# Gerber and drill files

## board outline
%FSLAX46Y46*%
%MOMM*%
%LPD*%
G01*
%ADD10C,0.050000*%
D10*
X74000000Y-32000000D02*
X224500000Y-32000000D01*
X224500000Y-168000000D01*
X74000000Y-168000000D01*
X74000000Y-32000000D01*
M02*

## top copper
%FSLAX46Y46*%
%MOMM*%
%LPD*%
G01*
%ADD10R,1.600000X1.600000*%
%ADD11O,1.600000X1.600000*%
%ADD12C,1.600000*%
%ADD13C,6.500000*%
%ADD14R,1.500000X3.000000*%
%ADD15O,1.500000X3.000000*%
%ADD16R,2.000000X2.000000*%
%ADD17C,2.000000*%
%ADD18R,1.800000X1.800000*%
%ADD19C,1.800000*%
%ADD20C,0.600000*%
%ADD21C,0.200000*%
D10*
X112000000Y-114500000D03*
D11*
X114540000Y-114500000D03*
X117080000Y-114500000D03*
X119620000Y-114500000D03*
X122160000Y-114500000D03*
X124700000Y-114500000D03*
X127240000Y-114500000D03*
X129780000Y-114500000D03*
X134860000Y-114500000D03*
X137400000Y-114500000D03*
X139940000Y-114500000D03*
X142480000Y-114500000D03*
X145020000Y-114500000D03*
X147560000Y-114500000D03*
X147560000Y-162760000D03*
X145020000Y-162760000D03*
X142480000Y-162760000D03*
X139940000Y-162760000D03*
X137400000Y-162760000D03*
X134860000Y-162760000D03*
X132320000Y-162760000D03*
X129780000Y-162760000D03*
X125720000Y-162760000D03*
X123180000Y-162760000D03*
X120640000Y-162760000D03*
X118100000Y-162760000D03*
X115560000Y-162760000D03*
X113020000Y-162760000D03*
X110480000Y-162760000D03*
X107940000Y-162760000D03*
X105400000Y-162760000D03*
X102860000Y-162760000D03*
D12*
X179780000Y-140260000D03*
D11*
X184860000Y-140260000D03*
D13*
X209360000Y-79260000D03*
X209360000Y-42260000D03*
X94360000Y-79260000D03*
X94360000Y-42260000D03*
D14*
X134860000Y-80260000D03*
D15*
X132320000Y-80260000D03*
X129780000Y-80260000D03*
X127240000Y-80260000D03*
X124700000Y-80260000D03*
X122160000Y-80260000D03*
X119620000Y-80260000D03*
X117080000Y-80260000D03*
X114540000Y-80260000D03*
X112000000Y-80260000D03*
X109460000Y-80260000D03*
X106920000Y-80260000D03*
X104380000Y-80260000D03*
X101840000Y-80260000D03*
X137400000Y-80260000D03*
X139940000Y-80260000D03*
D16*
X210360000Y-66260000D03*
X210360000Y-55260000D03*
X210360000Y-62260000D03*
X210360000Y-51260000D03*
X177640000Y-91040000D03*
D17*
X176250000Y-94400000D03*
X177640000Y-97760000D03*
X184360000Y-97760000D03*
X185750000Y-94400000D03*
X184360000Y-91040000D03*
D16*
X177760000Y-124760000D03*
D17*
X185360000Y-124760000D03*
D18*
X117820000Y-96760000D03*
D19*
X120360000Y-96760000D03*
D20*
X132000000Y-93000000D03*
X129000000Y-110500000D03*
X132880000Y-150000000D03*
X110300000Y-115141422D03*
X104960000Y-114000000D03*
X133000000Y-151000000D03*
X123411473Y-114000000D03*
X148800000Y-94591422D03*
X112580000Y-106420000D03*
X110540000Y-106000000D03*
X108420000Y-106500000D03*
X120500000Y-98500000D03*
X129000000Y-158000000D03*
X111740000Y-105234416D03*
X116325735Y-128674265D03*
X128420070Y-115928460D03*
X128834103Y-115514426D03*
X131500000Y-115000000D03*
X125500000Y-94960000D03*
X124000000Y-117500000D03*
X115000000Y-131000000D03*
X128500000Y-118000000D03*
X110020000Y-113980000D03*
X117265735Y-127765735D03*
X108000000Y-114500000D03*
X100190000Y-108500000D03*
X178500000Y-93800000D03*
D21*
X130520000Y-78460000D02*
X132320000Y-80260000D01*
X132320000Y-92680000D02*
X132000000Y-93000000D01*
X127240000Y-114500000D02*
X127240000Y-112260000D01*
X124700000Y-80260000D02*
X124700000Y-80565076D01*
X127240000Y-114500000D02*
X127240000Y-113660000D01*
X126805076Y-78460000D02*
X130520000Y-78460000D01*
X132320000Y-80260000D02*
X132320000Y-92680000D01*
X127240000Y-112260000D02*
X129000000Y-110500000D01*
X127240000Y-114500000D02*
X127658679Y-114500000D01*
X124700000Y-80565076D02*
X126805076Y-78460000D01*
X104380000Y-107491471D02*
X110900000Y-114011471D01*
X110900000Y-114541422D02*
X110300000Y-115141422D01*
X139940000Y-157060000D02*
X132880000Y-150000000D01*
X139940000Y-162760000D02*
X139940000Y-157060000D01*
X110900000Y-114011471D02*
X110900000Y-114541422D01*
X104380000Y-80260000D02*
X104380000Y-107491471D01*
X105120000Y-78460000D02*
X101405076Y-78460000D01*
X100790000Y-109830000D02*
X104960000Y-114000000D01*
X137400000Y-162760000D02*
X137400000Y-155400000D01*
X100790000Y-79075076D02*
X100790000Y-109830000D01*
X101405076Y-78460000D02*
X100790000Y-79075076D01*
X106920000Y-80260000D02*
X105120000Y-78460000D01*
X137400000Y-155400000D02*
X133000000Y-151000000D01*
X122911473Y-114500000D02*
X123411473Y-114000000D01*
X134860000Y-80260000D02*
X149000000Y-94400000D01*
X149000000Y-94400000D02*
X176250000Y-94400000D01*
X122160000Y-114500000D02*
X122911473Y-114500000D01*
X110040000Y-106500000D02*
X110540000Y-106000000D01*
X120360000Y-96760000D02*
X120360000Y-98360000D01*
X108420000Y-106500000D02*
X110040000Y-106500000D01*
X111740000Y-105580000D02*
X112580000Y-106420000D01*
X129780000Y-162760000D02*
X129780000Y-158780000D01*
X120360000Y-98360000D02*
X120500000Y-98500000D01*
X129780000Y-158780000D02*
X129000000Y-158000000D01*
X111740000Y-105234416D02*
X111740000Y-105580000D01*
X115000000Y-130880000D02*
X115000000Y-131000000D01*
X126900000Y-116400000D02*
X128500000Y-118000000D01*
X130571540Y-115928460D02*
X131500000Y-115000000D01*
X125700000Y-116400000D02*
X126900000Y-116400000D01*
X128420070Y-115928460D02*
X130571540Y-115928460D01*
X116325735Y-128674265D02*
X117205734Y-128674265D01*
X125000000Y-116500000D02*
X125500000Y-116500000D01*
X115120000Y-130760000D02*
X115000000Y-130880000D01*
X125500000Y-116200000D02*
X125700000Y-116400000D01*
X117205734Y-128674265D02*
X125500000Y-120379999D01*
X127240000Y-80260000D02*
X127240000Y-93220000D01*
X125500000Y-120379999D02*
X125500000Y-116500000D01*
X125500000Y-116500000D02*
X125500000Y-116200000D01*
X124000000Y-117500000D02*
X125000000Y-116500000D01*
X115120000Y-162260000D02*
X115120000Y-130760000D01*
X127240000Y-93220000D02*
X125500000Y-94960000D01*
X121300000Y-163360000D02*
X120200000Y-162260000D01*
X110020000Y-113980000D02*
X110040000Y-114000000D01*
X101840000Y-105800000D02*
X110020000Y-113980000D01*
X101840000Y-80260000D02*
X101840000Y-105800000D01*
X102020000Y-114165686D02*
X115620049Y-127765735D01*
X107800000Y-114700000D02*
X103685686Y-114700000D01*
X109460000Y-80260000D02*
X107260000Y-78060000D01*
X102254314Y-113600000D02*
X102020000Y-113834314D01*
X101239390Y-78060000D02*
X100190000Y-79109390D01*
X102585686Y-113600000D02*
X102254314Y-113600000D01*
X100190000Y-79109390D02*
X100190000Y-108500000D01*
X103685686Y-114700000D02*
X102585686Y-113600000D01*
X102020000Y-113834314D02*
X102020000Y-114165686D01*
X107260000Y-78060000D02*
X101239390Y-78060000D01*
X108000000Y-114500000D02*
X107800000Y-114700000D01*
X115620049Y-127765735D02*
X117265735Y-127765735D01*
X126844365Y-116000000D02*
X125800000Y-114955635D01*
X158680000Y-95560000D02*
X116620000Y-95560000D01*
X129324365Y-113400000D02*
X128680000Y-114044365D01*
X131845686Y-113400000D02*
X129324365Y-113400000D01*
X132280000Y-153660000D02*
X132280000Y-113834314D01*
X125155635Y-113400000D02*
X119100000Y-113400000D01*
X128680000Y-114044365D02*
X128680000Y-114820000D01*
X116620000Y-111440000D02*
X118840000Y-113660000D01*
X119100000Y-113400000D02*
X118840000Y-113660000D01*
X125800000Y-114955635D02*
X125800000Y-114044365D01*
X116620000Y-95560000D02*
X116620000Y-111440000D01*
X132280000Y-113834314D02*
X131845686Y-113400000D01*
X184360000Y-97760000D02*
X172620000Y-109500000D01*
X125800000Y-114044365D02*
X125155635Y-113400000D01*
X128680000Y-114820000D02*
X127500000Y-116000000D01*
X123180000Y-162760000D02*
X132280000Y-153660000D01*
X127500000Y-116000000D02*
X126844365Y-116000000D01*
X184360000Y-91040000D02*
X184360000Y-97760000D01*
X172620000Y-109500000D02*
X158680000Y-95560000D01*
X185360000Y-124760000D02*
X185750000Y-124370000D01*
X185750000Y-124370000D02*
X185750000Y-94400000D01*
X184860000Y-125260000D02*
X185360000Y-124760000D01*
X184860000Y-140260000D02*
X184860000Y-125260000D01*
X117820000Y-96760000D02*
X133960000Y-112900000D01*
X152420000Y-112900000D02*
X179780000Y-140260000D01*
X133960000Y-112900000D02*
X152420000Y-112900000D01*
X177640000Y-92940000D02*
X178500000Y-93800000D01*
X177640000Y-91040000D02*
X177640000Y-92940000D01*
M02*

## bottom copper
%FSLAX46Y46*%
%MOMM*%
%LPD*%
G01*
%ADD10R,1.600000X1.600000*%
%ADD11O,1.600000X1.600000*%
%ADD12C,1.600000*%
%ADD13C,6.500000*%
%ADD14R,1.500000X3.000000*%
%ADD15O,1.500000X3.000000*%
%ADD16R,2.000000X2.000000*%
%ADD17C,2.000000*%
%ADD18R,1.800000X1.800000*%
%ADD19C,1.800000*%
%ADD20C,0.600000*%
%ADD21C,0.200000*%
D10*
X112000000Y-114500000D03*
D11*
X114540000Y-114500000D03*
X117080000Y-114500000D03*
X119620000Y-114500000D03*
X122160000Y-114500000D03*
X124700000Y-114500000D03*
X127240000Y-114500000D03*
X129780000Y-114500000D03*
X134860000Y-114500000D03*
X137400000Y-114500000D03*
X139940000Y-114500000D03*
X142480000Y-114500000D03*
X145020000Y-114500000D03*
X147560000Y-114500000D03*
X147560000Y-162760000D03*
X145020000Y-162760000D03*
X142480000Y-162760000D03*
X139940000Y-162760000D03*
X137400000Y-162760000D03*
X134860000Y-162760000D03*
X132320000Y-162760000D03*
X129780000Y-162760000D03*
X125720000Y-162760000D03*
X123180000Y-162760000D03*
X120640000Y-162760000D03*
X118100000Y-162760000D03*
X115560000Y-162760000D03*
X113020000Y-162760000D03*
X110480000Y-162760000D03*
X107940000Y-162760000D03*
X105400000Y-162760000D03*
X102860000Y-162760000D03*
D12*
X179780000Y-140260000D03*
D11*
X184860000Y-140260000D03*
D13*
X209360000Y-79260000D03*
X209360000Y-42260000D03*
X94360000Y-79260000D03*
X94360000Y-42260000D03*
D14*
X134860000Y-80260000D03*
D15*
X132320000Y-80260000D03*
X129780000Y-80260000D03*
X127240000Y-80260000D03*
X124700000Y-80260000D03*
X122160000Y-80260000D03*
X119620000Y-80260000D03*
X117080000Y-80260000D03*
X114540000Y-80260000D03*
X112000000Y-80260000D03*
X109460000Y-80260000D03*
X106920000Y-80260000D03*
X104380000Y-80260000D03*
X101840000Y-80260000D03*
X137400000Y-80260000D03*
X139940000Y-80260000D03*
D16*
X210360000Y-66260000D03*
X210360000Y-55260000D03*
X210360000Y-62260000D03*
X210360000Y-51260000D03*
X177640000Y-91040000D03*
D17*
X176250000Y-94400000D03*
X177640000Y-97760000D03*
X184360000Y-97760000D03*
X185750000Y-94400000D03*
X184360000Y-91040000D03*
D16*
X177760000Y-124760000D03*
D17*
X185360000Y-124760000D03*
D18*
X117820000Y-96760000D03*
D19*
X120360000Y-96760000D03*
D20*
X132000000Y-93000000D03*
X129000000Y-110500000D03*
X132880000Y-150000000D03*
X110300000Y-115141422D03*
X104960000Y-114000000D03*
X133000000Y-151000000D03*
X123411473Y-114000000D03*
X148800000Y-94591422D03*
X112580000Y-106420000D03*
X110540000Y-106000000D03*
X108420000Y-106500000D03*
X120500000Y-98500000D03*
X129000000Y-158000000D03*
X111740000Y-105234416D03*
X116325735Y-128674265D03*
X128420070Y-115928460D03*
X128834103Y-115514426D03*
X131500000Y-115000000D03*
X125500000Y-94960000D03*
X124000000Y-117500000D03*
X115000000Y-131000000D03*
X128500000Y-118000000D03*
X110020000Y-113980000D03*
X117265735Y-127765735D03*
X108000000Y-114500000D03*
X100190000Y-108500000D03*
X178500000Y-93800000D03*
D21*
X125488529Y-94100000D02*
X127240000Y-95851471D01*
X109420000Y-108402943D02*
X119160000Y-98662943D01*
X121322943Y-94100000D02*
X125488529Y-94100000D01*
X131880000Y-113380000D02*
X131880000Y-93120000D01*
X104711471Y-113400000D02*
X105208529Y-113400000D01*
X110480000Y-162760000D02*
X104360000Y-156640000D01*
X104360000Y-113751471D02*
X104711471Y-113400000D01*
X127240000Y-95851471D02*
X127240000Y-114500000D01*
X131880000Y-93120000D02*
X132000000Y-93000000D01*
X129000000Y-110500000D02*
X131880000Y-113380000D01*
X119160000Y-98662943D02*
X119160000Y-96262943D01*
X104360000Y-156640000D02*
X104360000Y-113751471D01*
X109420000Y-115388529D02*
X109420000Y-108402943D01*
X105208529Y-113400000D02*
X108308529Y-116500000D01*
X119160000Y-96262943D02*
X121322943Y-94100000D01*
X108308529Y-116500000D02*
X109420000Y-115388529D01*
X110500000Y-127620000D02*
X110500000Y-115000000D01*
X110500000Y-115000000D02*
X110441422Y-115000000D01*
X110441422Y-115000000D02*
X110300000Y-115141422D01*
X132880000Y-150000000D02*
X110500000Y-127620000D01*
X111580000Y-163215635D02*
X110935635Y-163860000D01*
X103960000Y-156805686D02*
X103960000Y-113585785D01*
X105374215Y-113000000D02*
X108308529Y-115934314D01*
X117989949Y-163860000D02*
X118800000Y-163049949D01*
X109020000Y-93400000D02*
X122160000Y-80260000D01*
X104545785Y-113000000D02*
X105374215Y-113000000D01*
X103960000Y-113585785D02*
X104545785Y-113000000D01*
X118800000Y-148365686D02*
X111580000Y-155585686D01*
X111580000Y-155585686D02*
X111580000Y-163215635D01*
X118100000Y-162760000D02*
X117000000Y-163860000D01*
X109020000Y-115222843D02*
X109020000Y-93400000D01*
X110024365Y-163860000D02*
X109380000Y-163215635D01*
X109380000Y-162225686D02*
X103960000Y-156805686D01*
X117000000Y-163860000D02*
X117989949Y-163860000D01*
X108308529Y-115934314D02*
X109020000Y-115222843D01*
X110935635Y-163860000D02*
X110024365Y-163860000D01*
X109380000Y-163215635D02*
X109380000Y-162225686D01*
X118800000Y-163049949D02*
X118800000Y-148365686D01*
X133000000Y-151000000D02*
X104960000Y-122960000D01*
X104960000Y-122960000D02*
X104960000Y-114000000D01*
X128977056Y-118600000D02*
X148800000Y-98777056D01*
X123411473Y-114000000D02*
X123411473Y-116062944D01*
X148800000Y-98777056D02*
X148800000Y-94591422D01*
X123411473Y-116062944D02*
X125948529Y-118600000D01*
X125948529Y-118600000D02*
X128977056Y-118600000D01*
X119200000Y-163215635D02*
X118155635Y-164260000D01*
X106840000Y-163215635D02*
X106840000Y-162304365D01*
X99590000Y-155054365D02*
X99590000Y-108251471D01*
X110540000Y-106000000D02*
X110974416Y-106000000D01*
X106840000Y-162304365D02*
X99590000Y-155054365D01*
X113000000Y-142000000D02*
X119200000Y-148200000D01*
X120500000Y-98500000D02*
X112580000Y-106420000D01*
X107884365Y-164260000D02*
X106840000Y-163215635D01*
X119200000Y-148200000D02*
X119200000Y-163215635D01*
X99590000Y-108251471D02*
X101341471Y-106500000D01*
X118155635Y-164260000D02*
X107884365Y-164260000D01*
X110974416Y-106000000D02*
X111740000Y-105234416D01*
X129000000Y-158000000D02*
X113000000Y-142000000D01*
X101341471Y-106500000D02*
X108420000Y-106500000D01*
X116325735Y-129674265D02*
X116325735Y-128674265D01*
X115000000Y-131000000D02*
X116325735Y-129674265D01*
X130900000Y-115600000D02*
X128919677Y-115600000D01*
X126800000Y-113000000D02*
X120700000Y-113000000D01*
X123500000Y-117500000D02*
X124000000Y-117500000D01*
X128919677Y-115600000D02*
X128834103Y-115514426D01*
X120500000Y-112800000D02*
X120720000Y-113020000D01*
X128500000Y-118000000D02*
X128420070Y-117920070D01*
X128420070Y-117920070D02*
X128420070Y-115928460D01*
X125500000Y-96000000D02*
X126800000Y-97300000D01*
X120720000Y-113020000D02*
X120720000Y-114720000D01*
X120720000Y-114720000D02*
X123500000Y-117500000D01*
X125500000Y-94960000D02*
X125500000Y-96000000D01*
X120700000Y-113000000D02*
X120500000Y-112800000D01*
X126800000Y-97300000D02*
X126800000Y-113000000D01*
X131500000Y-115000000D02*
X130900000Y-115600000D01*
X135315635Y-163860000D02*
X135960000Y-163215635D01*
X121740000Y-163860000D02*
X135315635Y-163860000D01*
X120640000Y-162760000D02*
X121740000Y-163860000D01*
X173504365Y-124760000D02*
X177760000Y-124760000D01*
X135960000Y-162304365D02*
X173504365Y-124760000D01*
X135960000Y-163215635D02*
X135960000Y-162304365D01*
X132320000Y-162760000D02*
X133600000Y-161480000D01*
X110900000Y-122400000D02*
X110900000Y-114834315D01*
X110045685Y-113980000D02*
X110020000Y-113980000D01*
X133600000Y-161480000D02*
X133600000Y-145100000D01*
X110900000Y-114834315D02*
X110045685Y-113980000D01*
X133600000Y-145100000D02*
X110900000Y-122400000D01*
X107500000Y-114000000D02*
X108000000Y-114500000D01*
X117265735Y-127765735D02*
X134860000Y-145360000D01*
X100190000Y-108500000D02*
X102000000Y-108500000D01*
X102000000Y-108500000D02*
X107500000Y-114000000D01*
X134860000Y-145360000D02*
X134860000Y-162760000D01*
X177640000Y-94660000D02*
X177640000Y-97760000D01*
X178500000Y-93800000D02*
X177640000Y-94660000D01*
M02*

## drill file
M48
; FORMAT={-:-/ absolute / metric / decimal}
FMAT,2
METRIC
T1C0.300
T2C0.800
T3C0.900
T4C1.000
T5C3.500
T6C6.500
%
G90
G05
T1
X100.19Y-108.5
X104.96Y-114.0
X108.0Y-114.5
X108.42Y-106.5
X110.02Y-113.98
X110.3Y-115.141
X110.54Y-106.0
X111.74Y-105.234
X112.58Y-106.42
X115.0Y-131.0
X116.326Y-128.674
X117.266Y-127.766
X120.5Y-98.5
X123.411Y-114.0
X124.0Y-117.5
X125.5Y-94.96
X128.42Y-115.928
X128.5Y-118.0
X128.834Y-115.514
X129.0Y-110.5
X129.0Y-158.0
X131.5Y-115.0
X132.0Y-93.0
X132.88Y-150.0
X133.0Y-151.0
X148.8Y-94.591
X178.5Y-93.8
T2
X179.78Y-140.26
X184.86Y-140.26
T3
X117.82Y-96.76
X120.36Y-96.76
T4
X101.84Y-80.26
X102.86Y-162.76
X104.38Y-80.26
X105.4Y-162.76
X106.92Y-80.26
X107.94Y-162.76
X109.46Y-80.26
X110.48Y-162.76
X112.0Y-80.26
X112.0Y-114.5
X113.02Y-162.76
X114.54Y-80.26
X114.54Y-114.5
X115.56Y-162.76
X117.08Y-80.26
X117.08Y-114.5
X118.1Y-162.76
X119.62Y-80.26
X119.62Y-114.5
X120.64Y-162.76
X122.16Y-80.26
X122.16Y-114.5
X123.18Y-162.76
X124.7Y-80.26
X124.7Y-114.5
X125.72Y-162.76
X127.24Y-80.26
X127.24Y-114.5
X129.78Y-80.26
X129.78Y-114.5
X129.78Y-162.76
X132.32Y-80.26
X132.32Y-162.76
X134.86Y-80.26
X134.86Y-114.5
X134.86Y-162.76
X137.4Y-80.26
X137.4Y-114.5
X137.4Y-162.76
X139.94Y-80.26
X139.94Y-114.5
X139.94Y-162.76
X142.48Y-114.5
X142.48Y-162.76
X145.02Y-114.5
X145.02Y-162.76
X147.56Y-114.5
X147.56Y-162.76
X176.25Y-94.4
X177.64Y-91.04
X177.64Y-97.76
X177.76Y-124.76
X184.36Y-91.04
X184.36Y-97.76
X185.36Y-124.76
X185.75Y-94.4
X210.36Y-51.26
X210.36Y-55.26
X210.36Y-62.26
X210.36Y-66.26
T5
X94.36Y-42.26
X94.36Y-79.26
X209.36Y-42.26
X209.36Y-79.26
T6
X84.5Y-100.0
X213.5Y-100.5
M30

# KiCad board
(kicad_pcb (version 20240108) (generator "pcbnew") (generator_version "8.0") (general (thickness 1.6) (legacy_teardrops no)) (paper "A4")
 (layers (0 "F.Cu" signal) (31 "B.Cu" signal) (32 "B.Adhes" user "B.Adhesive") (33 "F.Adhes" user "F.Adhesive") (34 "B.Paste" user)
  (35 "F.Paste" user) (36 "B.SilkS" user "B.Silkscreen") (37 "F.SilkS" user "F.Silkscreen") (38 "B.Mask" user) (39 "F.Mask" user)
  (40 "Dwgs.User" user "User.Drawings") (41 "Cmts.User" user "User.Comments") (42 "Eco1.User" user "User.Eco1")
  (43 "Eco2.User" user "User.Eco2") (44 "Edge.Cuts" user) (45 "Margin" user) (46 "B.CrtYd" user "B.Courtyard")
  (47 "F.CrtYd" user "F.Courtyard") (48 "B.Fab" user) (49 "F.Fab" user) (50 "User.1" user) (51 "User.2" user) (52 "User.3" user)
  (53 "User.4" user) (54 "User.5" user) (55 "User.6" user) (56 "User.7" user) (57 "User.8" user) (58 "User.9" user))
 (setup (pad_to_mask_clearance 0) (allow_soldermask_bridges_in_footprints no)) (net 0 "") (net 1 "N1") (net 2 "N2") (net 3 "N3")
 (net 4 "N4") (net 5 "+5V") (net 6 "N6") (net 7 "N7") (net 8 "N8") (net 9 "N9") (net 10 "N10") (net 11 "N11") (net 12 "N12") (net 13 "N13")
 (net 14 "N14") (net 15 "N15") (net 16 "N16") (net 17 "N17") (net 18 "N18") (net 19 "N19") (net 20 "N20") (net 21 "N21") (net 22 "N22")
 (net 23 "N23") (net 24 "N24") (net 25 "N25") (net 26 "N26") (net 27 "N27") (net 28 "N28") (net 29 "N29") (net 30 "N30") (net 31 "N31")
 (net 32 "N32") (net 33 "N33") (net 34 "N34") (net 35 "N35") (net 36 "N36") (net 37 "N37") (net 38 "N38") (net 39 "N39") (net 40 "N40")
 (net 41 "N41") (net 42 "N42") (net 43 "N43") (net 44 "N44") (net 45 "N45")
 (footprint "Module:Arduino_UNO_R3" (layer "F.Cu") (at 112 114.5)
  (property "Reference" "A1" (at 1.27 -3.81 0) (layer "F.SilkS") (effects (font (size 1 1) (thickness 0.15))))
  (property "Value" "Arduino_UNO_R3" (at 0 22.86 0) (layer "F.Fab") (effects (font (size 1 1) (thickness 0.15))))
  (pad "1" thru_hole rect (at 0 0 90) (size 1.6 1.6) (drill 1) (layers "*.Cu" "*.Mask") (remove_unused_layers no) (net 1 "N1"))
  (pad "2" thru_hole oval (at 2.54 0 90) (size 1.6 1.6) (drill 1) (layers "*.Cu" "*.Mask") (remove_unused_layers no) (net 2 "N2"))
  (pad "3" thru_hole oval (at 5.08 0 90) (size 1.6 1.6) (drill 1) (layers "*.Cu" "*.Mask") (remove_unused_layers no) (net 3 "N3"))
  (pad "4" thru_hole oval (at 7.62 0 90) (size 1.6 1.6) (drill 1) (layers "*.Cu" "*.Mask") (remove_unused_layers no) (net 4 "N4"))
  (pad "5" thru_hole oval (at 10.16 0 90) (size 1.6 1.6) (drill 1) (layers "*.Cu" "*.Mask") (remove_unused_layers no) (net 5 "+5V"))
  (pad "6" thru_hole oval (at 12.7 0 90) (size 1.6 1.6) (drill 1) (layers "*.Cu" "*.Mask") (remove_unused_layers no) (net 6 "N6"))
  (pad "7" thru_hole oval (at 15.24 0 90) (size 1.6 1.6) (drill 1) (layers "*.Cu" "*.Mask") (remove_unused_layers no) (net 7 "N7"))
  (pad "8" thru_hole oval (at 17.78 0 90) (size 1.6 1.6) (drill 1) (layers "*.Cu" "*.Mask") (remove_unused_layers no) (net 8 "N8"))
  (pad "9" thru_hole oval (at 22.86 0 90) (size 1.6 1.6) (drill 1) (layers "*.Cu" "*.Mask") (remove_unused_layers no) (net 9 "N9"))
  (pad "10" thru_hole oval (at 25.4 0 90) (size 1.6 1.6) (drill 1) (layers "*.Cu" "*.Mask") (remove_unused_layers no) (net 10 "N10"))
  (pad "11" thru_hole oval (at 27.94 0 90) (size 1.6 1.6) (drill 1) (layers "*.Cu" "*.Mask") (remove_unused_layers no) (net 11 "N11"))
  (pad "12" thru_hole oval (at 30.48 0 90) (size 1.6 1.6) (drill 1) (layers "*.Cu" "*.Mask") (remove_unused_layers no) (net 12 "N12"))
  (pad "13" thru_hole oval (at 33.02 0 90) (size 1.6 1.6) (drill 1) (layers "*.Cu" "*.Mask") (remove_unused_layers no) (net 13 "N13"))
  (pad "14" thru_hole oval (at 35.56 0 90) (size 1.6 1.6) (drill 1) (layers "*.Cu" "*.Mask") (remove_unused_layers no) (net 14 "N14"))
  (pad "15" thru_hole oval (at 35.56 48.26 90) (size 1.6 1.6) (drill 1) (layers "*.Cu" "*.Mask") (remove_unused_layers no) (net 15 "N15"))
  (pad "16" thru_hole oval (at 33.02 48.26 90) (size 1.6 1.6) (drill 1) (layers "*.Cu" "*.Mask") (remove_unused_layers no) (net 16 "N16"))
  (pad "17" thru_hole oval (at 30.48 48.26 90) (size 1.6 1.6) (drill 1) (layers "*.Cu" "*.Mask") (remove_unused_layers no) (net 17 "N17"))
  (pad "18" thru_hole oval (at 27.94 48.26 90) (size 1.6 1.6) (drill 1) (layers "*.Cu" "*.Mask") (remove_unused_layers no) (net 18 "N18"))
  (pad "19" thru_hole oval (at 25.4 48.26 90) (size 1.6 1.6) (drill 1) (layers "*.Cu" "*.Mask") (remove_unused_layers no) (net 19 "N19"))
  (pad "20" thru_hole oval (at 22.86 48.26 90) (size 1.6 1.6) (drill 1) (layers "*.Cu" "*.Mask") (remove_unused_layers no) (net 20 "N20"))
  (pad "21" thru_hole oval (at 20.32 48.26 90) (size 1.6 1.6) (drill 1) (layers "*.Cu" "*.Mask") (remove_unused_layers no) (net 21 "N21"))
  (pad "22" thru_hole oval (at 17.78 48.26 90) (size 1.6 1.6) (drill 1) (layers "*.Cu" "*.Mask") (remove_unused_layers no) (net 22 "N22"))
  (pad "23" thru_hole oval (at 13.72 48.26 90) (size 1.6 1.6) (drill 1) (layers "*.Cu" "*.Mask") (remove_unused_layers no) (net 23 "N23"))
  (pad "24" thru_hole oval (at 11.18 48.26 90) (size 1.6 1.6) (drill 1) (layers "*.Cu" "*.Mask") (remove_unused_layers no) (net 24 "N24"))
  (pad "25" thru_hole oval (at 8.64 48.26 90) (size 1.6 1.6) (drill 1) (layers "*.Cu" "*.Mask") (remove_unused_layers no) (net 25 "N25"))
  (pad "26" thru_hole oval (at 6.1 48.26 90) (size 1.6 1.6) (drill 1) (layers "*.Cu" "*.Mask") (remove_unused_layers no) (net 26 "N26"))
  (pad "27" thru_hole oval (at 3.56 48.26 90) (size 1.6 1.6) (drill 1) (layers "*.Cu" "*.Mask") (remove_unused_layers no) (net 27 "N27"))
  (pad "28" thru_hole oval (at 1.02 48.26 90) (size 1.6 1.6) (drill 1) (layers "*.Cu" "*.Mask") (remove_unused_layers no) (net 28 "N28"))
  (pad "29" thru_hole oval (at -1.52 48.26 90) (size 1.6 1.6) (drill 1) (layers "*.Cu" "*.Mask") (remove_unused_layers no) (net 7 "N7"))
  (pad "30" thru_hole oval (at -4.06 48.26 90) (size 1.6 1.6) (drill 1) (layers "*.Cu" "*.Mask") (remove_unused_layers no) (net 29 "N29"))
  (pad "31" thru_hole oval (at -6.6 48.26 90) (size 1.6 1.6) (drill 1) (layers "*.Cu" "*.Mask") (remove_unused_layers no) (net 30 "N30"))
  (pad "32" thru_hole oval (at -9.14 48.26 90) (size 1.6 1.6) (drill 1) (layers "*.Cu" "*.Mask") (remove_unused_layers no) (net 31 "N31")))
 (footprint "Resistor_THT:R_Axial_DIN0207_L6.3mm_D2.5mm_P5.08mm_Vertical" (layer "F.Cu") (at 179.78 140.26)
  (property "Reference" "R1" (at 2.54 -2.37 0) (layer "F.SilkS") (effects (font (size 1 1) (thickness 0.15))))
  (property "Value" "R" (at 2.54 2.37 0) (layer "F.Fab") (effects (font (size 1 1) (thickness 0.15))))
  (pad "1" thru_hole circle (at 0 0) (size 1.6 1.6) (drill 0.8) (layers "*.Cu" "*.Mask") (remove_unused_layers no) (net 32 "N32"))
  (pad "2" thru_hole oval (at 5.08 0) (size 1.6 1.6) (drill 0.8) (layers "*.Cu" "*.Mask") (remove_unused_layers no) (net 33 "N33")))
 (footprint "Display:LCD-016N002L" (layer "F.Cu") (at 134.86 80.26 180)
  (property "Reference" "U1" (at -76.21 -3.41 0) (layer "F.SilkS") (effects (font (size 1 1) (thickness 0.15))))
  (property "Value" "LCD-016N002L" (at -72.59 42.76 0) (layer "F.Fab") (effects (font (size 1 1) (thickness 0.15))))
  (pad "" thru_hole circle (at -74.5 1) (size 6.5 6.5) (drill 3.5) (layers "*.Cu" "*.Mask") (remove_unused_layers no))
  (pad "" thru_hole circle (at -74.5 38) (size 6.5 6.5) (drill 3.5) (layers "*.Cu" "*.Mask") (remove_unused_layers no))
  (pad "" thru_hole circle (at 40.5 1) (size 6.5 6.5) (drill 3.5) (layers "*.Cu" "*.Mask") (remove_unused_layers no))
  (pad "" thru_hole circle (at 40.5 38) (size 6.5 6.5) (drill 3.5) (layers "*.Cu" "*.Mask") (remove_unused_layers no))
  (pad "1" thru_hole rect (at 0 0) (size 1.5 3) (drill 1) (layers "*.Cu" "*.Mask") (remove_unused_layers no) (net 5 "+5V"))
  (pad "2" thru_hole oval (at 2.54 0) (size 1.5 3) (drill 1) (layers "*.Cu" "*.Mask") (remove_unused_layers no) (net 7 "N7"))
  (pad "3" thru_hole oval (at 5.08 0) (size 1.5 3) (drill 1) (layers "*.Cu" "*.Mask") (remove_unused_layers no) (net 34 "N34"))
  (pad "4" thru_hole oval (at 7.62 0) (size 1.5 3) (drill 1) (layers "*.Cu" "*.Mask") (remove_unused_layers no) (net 27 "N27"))
  (pad "5" thru_hole oval (at 10.16 0) (size 1.5 3) (drill 1) (layers "*.Cu" "*.Mask") (remove_unused_layers no) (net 7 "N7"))
  (pad "6" thru_hole oval (at 12.7 0) (size 1.5 3) (drill 1) (layers "*.Cu" "*.Mask") (remove_unused_layers no) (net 26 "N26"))
  (pad "7" thru_hole oval (at 15.24 0) (size 1.5 3) (drill 1) (layers "*.Cu" "*.Mask") (remove_unused_layers no) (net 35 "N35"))
  (pad "8" thru_hole oval (at 17.78 0) (size 1.5 3) (drill 1) (layers "*.Cu" "*.Mask") (remove_unused_layers no) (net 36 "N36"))
  (pad "9" thru_hole oval (at 20.32 0) (size 1.5 3) (drill 1) (layers "*.Cu" "*.Mask") (remove_unused_layers no) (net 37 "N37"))
  (pad "10" thru_hole oval (at 22.86 0) (size 1.5 3) (drill 1) (layers "*.Cu" "*.Mask") (remove_unused_layers no) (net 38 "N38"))
  (pad "11" thru_hole oval (at 25.4 0) (size 1.5 3) (drill 1) (layers "*.Cu" "*.Mask") (remove_unused_layers no) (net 20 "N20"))
  (pad "12" thru_hole oval (at 27.94 0) (size 1.5 3) (drill 1) (layers "*.Cu" "*.Mask") (remove_unused_layers no) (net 19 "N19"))
  (pad "13" thru_hole oval (at 30.48 0) (size 1.5 3) (drill 1) (layers "*.Cu" "*.Mask") (remove_unused_layers no) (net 18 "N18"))
  (pad "14" thru_hole oval (at 33.02 0) (size 1.5 3) (drill 1) (layers "*.Cu" "*.Mask") (remove_unused_layers no) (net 21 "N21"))
  (pad "15" thru_hole oval (at -2.54 0) (size 1.5 3) (drill 1) (layers "*.Cu" "*.Mask") (remove_unused_layers no) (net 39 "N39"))
  (pad "16" thru_hole oval (at -5.08 0) (size 1.5 3) (drill 1) (layers "*.Cu" "*.Mask") (remove_unused_layers no) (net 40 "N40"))
  (pad "A1" thru_hole rect (at -75.5 14) (size 2 2) (drill 1) (layers "*.Cu" "*.Mask") (remove_unused_layers no) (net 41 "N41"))
  (pad "A2" thru_hole rect (at -75.5 25) (size 2 2) (drill 1) (layers "*.Cu" "*.Mask") (remove_unused_layers no) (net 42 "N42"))
  (pad "K1" thru_hole rect (at -75.5 18) (size 2 2) (drill 1) (layers "*.Cu" "*.Mask") (remove_unused_layers no) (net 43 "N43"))
  (pad "K2" thru_hole rect (at -75.5 29) (size 2 2) (drill 1) (layers "*.Cu" "*.Mask") (remove_unused_layers no) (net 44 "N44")))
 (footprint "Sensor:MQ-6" (layer "F.Cu") (at 177.64 91.04)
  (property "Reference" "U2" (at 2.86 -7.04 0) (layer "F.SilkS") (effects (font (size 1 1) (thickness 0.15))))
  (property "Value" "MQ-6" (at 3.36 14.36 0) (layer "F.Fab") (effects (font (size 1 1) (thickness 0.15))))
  (pad "1" thru_hole rect (at 0 0) (size 2 2) (drill 1) (layers "*.Cu" "*.Mask") (remove_unused_layers no) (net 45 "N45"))
  (pad "2" thru_hole circle (at -1.39 3.36) (size 2 2) (drill 1) (layers "*.Cu" "*.Mask") (remove_unused_layers no) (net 5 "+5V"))
  (pad "3" thru_hole circle (at 0 6.72 90) (size 2 2) (drill 1) (layers "*.Cu" "*.Mask") (remove_unused_layers no) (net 45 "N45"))
  (pad "4" thru_hole circle (at 6.72 6.72 180) (size 2 2) (drill 1) (layers "*.Cu" "*.Mask") (remove_unused_layers no) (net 24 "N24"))
  (pad "5" thru_hole circle (at 8.11 3.36) (size 2 2) (drill 1) (layers "*.Cu" "*.Mask") (remove_unused_layers no) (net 33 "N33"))
  (pad "6" thru_hole circle (at 6.72 0 270) (size 2 2) (drill 1) (layers "*.Cu" "*.Mask") (remove_unused_layers no) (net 24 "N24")))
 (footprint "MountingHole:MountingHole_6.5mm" (layer "F.Cu") (at 213.5 100.5)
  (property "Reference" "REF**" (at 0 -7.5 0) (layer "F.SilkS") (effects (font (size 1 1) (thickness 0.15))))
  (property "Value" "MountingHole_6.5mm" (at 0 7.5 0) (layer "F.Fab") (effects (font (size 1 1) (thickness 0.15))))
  (pad "" np_thru_hole circle (at 0 0) (size 6.5 6.5) (drill 6.5) (layers "*.Cu" "*.Mask")))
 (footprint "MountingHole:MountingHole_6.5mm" (layer "F.Cu") (at 84.5 100)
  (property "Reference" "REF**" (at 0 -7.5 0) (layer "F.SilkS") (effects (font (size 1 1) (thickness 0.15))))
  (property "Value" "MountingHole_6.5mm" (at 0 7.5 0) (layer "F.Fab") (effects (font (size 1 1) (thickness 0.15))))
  (pad "" np_thru_hole circle (at 0 0) (size 6.5 6.5) (drill 6.5) (layers "*.Cu" "*.Mask")))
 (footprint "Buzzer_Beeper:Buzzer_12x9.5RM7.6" (layer "F.Cu") (at 177.76 124.76)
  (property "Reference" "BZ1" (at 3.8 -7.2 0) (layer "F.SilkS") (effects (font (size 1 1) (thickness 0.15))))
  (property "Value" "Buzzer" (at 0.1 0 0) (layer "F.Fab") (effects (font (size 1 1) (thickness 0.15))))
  (pad "1" thru_hole rect (at 0 0) (size 2 2) (drill 1) (layers "*.Cu" "*.Mask") (remove_unused_layers no) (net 25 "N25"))
  (pad "2" thru_hole circle (at 7.6 0) (size 2 2) (drill 1) (layers "*.Cu" "*.Mask") (remove_unused_layers no) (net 33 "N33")))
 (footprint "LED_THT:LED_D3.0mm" (layer "F.Cu") (at 117.82 96.76)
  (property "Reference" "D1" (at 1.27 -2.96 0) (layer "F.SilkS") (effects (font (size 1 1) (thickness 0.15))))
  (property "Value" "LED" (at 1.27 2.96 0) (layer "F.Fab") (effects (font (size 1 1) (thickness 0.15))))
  (pad "1" thru_hole rect (at 0 0) (size 1.8 1.8) (drill 0.9) (layers "*.Cu" "*.Mask") (remove_unused_layers no) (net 32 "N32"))
  (pad "2" thru_hole circle (at 2.54 0) (size 1.8 1.8) (drill 0.9) (layers "*.Cu" "*.Mask") (remove_unused_layers no) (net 22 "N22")))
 (gr_rect (start 74 32) (end 224.5 168) (stroke (width 0.05) (type default)) (fill none) (layer "Edge.Cuts"))
 (segment (start 130.52 78.46) (end 132.32 80.26) (width 0.2) (layer "F.Cu") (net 7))
 (segment (start 132.32 92.68) (end 132 93) (width 0.2) (layer "F.Cu") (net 7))
 (segment (start 127.24 114.5) (end 127.24 112.26) (width 0.2) (layer "F.Cu") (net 7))
 (segment (start 124.7 80.26) (end 124.7 80.565076) (width 0.2) (layer "F.Cu") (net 7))
 (segment (start 127.24 114.5) (end 127.24 113.66) (width 0.2) (layer "F.Cu") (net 7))
 (segment (start 126.805076 78.46) (end 130.52 78.46) (width 0.2) (layer "F.Cu") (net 7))
 (segment (start 132.32 80.26) (end 132.32 92.68) (width 0.2) (layer "F.Cu") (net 7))
 (segment (start 127.24 112.26) (end 129 110.5) (width 0.2) (layer "F.Cu") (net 7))
 (segment (start 127.24 114.5) (end 127.658679 114.5) (width 0.2) (layer "F.Cu") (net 7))
 (segment (start 124.7 80.565076) (end 126.805076 78.46) (width 0.2) (layer "F.Cu") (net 7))
 (via (at 132 93) (size 0.6) (drill 0.3) (layers "F.Cu" "B.Cu") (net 7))
 (via (at 129 110.5) (size 0.6) (drill 0.3) (layers "F.Cu" "B.Cu") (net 7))
 (segment (start 125.488529 94.1) (end 127.24 95.851471) (width 0.2) (layer "B.Cu") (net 7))
 (segment (start 109.42 108.402943) (end 119.16 98.662943) (width 0.2) (layer "B.Cu") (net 7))
 (segment (start 121.322943 94.1) (end 125.488529 94.1) (width 0.2) (layer "B.Cu") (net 7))
 (segment (start 131.88 113.38) (end 131.88 93.12) (width 0.2) (layer "B.Cu") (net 7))
 (segment (start 104.711471 113.4) (end 105.208529 113.4) (width 0.2) (layer "B.Cu") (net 7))
 (segment (start 110.48 162.76) (end 104.36 156.64) (width 0.2) (layer "B.Cu") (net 7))
 (segment (start 104.36 113.751471) (end 104.711471 113.4) (width 0.2) (layer "B.Cu") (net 7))
 (segment (start 127.24 95.851471) (end 127.24 114.5) (width 0.2) (layer "B.Cu") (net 7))
 (segment (start 131.88 93.12) (end 132 93) (width 0.2) (layer "B.Cu") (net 7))
 (segment (start 129 110.5) (end 131.88 113.38) (width 0.2) (layer "B.Cu") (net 7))
 (segment (start 119.16 98.662943) (end 119.16 96.262943) (width 0.2) (layer "B.Cu") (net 7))
 (segment (start 104.36 156.64) (end 104.36 113.751471) (width 0.2) (layer "B.Cu") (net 7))
 (segment (start 109.42 115.388529) (end 109.42 108.402943) (width 0.2) (layer "B.Cu") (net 7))
 (segment (start 105.208529 113.4) (end 108.308529 116.5) (width 0.2) (layer "B.Cu") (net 7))
 (segment (start 119.16 96.262943) (end 121.322943 94.1) (width 0.2) (layer "B.Cu") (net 7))
 (segment (start 108.308529 116.5) (end 109.42 115.388529) (width 0.2) (layer "B.Cu") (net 7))
 (segment (start 104.38 107.491471) (end 110.9 114.011471) (width 0.2) (layer "F.Cu") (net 18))
 (segment (start 110.9 114.541422) (end 110.3 115.141422) (width 0.2) (layer "F.Cu") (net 18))
 (segment (start 139.94 157.06) (end 132.88 150) (width 0.2) (layer "F.Cu") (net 18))
 (segment (start 139.94 162.76) (end 139.94 157.06) (width 0.2) (layer "F.Cu") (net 18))
 (segment (start 110.9 114.011471) (end 110.9 114.541422) (width 0.2) (layer "F.Cu") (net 18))
 (segment (start 104.38 80.26) (end 104.38 107.491471) (width 0.2) (layer "F.Cu") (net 18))
 (via (at 132.88 150) (size 0.6) (drill 0.3) (layers "F.Cu" "B.Cu") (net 18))
 (via (at 110.3 115.141422) (size 0.6) (drill 0.3) (layers "F.Cu" "B.Cu") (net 18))
 (segment (start 110.5 127.62) (end 110.5 115) (width 0.2) (layer "B.Cu") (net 18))
 (segment (start 110.5 115) (end 110.441422 115) (width 0.2) (layer "B.Cu") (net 18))
 (segment (start 110.441422 115) (end 110.3 115.141422) (width 0.2) (layer "B.Cu") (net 18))
 (segment (start 132.88 150) (end 110.5 127.62) (width 0.2) (layer "B.Cu") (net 18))
 (segment (start 111.58 163.215635) (end 110.935635 163.86) (width 0.2) (layer "B.Cu") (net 26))
 (segment (start 103.96 156.805686) (end 103.96 113.585785) (width 0.2) (layer "B.Cu") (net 26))
 (segment (start 105.374215 113) (end 108.308529 115.934314) (width 0.2) (layer "B.Cu") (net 26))
 (segment (start 117.989949 163.86) (end 118.8 163.049949) (width 0.2) (layer "B.Cu") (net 26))
 (segment (start 109.02 93.4) (end 122.16 80.26) (width 0.2) (layer "B.Cu") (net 26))
 (segment (start 104.545785 113) (end 105.374215 113) (width 0.2) (layer "B.Cu") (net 26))
 (segment (start 103.96 113.585785) (end 104.545785 113) (width 0.2) (layer "B.Cu") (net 26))
 (segment (start 118.8 148.365686) (end 111.58 155.585686) (width 0.2) (layer "B.Cu") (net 26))
 (segment (start 111.58 155.585686) (end 111.58 163.215635) (width 0.2) (layer "B.Cu") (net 26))
 (segment (start 118.1 162.76) (end 117 163.86) (width 0.2) (layer "B.Cu") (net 26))
 (segment (start 109.02 115.222843) (end 109.02 93.4) (width 0.2) (layer "B.Cu") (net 26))
 (segment (start 110.024365 163.86) (end 109.38 163.215635) (width 0.2) (layer "B.Cu") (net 26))
 (segment (start 109.38 162.225686) (end 103.96 156.805686) (width 0.2) (layer "B.Cu") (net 26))
 (segment (start 117 163.86) (end 117.989949 163.86) (width 0.2) (layer "B.Cu") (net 26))
 (segment (start 108.308529 115.934314) (end 109.02 115.222843) (width 0.2) (layer "B.Cu") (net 26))
 (segment (start 110.935635 163.86) (end 110.024365 163.86) (width 0.2) (layer "B.Cu") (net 26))
 (segment (start 109.38 163.215635) (end 109.38 162.225686) (width 0.2) (layer "B.Cu") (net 26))
 (segment (start 118.8 163.049949) (end 118.8 148.365686) (width 0.2) (layer "B.Cu") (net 26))
 (segment (start 105.12 78.46) (end 101.405076 78.46) (width 0.2) (layer "F.Cu") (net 19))
 (segment (start 100.79 109.83) (end 104.96 114) (width 0.2) (layer "F.Cu") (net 19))
 (segment (start 137.4 162.76) (end 137.4 155.4) (width 0.2) (layer "F.Cu") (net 19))
 (segment (start 100.79 79.075076) (end 100.79 109.83) (width 0.2) (layer "F.Cu") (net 19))
 (segment (start 101.405076 78.46) (end 100.79 79.075076) (width 0.2) (layer "F.Cu") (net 19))
 (segment (start 106.92 80.26) (end 105.12 78.46) (width 0.2) (layer "F.Cu") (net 19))
 (segment (start 137.4 155.4) (end 133 151) (width 0.2) (layer "F.Cu") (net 19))
 (via (at 104.96 114) (size 0.6) (drill 0.3) (layers "F.Cu" "B.Cu") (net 19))
 (via (at 133 151) (size 0.6) (drill 0.3) (layers "F.Cu" "B.Cu") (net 19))
 (segment (start 133 151) (end 104.96 122.96) (width 0.2) (layer "B.Cu") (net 19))
 (segment (start 104.96 122.96) (end 104.96 114) (width 0.2) (layer "B.Cu") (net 19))
 (segment (start 122.911473 114.5) (end 123.411473 114) (width 0.2) (layer "F.Cu") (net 5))
 (segment (start 134.86 80.26) (end 149 94.4) (width 0.2) (layer "F.Cu") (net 5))
 (segment (start 149 94.4) (end 176.25 94.4) (width 0.2) (layer "F.Cu") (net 5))
 (segment (start 122.16 114.5) (end 122.911473 114.5) (width 0.2) (layer "F.Cu") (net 5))
 (via (at 123.411473 114) (size 0.6) (drill 0.3) (layers "F.Cu" "B.Cu") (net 5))
 (via (at 148.8 94.591422) (size 0.6) (drill 0.3) (layers "F.Cu" "B.Cu") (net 5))
 (segment (start 128.977056 118.6) (end 148.8 98.777056) (width 0.2) (layer "B.Cu") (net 5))
 (segment (start 123.411473 114) (end 123.411473 116.062944) (width 0.2) (layer "B.Cu") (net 5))
 (segment (start 148.8 98.777056) (end 148.8 94.591422) (width 0.2) (layer "B.Cu") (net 5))
 (segment (start 123.411473 116.062944) (end 125.948529 118.6) (width 0.2) (layer "B.Cu") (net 5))
 (segment (start 125.948529 118.6) (end 128.977056 118.6) (width 0.2) (layer "B.Cu") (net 5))
 (segment (start 110.04 106.5) (end 110.54 106) (width 0.2) (layer "F.Cu") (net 22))
 (segment (start 120.36 96.76) (end 120.36 98.36) (width 0.2) (layer "F.Cu") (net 22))
 (segment (start 108.42 106.5) (end 110.04 106.5) (width 0.2) (layer "F.Cu") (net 22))
 (segment (start 111.74 105.58) (end 112.58 106.42) (width 0.2) (layer "F.Cu") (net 22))
 (segment (start 129.78 162.76) (end 129.78 158.78) (width 0.2) (layer "F.Cu") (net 22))
 (segment (start 120.36 98.36) (end 120.5 98.5) (width 0.2) (layer "F.Cu") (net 22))
 (segment (start 129.78 158.78) (end 129 158) (width 0.2) (layer "F.Cu") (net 22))
 (segment (start 111.74 105.234416) (end 111.74 105.58) (width 0.2) (layer "F.Cu") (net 22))
 (via (at 112.58 106.42) (size 0.6) (drill 0.3) (layers "F.Cu" "B.Cu") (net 22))
 (via (at 110.54 106) (size 0.6) (drill 0.3) (layers "F.Cu" "B.Cu") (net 22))
 (via (at 108.42 106.5) (size 0.6) (drill 0.3) (layers "F.Cu" "B.Cu") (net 22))
 (via (at 120.5 98.5) (size 0.6) (drill 0.3) (layers "F.Cu" "B.Cu") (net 22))
 (via (at 129 158) (size 0.6) (drill 0.3) (layers "F.Cu" "B.Cu") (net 22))
 (via (at 111.74 105.234416) (size 0.6) (drill 0.3) (layers "F.Cu" "B.Cu") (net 22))
 (segment (start 119.2 163.215635) (end 118.155635 164.26) (width 0.2) (layer "B.Cu") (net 22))
 (segment (start 106.84 163.215635) (end 106.84 162.304365) (width 0.2) (layer "B.Cu") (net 22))
 (segment (start 99.59 155.054365) (end 99.59 108.251471) (width 0.2) (layer "B.Cu") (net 22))
 (segment (start 110.54 106) (end 110.974416 106) (width 0.2) (layer "B.Cu") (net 22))
 (segment (start 106.84 162.304365) (end 99.59 155.054365) (width 0.2) (layer "B.Cu") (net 22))
 (segment (start 113 142) (end 119.2 148.2) (width 0.2) (layer "B.Cu") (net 22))
 (segment (start 120.5 98.5) (end 112.58 106.42) (width 0.2) (layer "B.Cu") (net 22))
 (segment (start 107.884365 164.26) (end 106.84 163.215635) (width 0.2) (layer "B.Cu") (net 22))
 (segment (start 119.2 148.2) (end 119.2 163.215635) (width 0.2) (layer "B.Cu") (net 22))
 (segment (start 99.59 108.251471) (end 101.341471 106.5) (width 0.2) (layer "B.Cu") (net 22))
 (segment (start 118.155635 164.26) (end 107.884365 164.26) (width 0.2) (layer "B.Cu") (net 22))
 (segment (start 110.974416 106) (end 111.74 105.234416) (width 0.2) (layer "B.Cu") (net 22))
 (segment (start 129 158) (end 113 142) (width 0.2) (layer "B.Cu") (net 22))
 (segment (start 101.341471 106.5) (end 108.42 106.5) (width 0.2) (layer "B.Cu") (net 22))
 (segment (start 115 130.88) (end 115 131) (width 0.2) (layer "F.Cu") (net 27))
 (segment (start 126.9 116.4) (end 128.5 118) (width 0.2) (layer "F.Cu") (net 27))
 (segment (start 130.57154 115.92846) (end 131.5 115) (width 0.2) (layer "F.Cu") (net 27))
 (segment (start 125.7 116.4) (end 126.9 116.4) (width 0.2) (layer "F.Cu") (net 27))
 (segment (start 128.42007 115.92846) (end 130.57154 115.92846) (width 0.2) (layer "F.Cu") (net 27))
 (segment (start 116.325735 128.674265) (end 117.205734 128.674265) (width 0.2) (layer "F.Cu") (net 27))
 (segment (start 125 116.5) (end 125.5 116.5) (width 0.2) (layer "F.Cu") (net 27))
 (segment (start 115.12 130.76) (end 115 130.88) (width 0.2) (layer "F.Cu") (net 27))
 (segment (start 125.5 116.2) (end 125.7 116.4) (width 0.2) (layer "F.Cu") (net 27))
 (segment (start 117.205734 128.674265) (end 125.5 120.379999) (width 0.2) (layer "F.Cu") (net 27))
 (segment (start 127.24 80.26) (end 127.24 93.22) (width 0.2) (layer "F.Cu") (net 27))
 (segment (start 125.5 120.379999) (end 125.5 116.5) (width 0.2) (layer "F.Cu") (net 27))
 (segment (start 125.5 116.5) (end 125.5 116.2) (width 0.2) (layer "F.Cu") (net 27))
 (segment (start 124 117.5) (end 125 116.5) (width 0.2) (layer "F.Cu") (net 27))
 (segment (start 115.12 162.26) (end 115.12 130.76) (width 0.2) (layer "F.Cu") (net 27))
 (segment (start 127.24 93.22) (end 125.5 94.96) (width 0.2) (layer "F.Cu") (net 27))
 (via (at 116.325735 128.674265) (size 0.6) (drill 0.3) (layers "F.Cu" "B.Cu") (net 27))
 (via (at 128.42007 115.92846) (size 0.6) (drill 0.3) (layers "F.Cu" "B.Cu") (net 27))
 (via (at 128.834103 115.514426) (size 0.6) (drill 0.3) (layers "F.Cu" "B.Cu") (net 27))
 (via (at 131.5 115) (size 0.6) (drill 0.3) (layers "F.Cu" "B.Cu") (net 27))
 (via (at 125.5 94.96) (size 0.6) (drill 0.3) (layers "F.Cu" "B.Cu") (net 27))
 (via (at 124 117.5) (size 0.6) (drill 0.3) (layers "F.Cu" "B.Cu") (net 27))
 (via (at 115 131) (size 0.6) (drill 0.3) (layers "F.Cu" "B.Cu") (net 27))
 (via (at 128.5 118) (size 0.6) (drill 0.3) (layers "F.Cu" "B.Cu") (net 27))
 (segment (start 116.325735 129.674265) (end 116.325735 128.674265) (width 0.2) (layer "B.Cu") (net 27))
 (segment (start 115 131) (end 116.325735 129.674265) (width 0.2) (layer "B.Cu") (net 27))
 (segment (start 130.9 115.6) (end 128.919677 115.6) (width 0.2) (layer "B.Cu") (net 27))
 (segment (start 126.8 113) (end 120.7 113) (width 0.2) (layer "B.Cu") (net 27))
 (segment (start 123.5 117.5) (end 124 117.5) (width 0.2) (layer "B.Cu") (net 27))
 (segment (start 128.919677 115.6) (end 128.834103 115.514426) (width 0.2) (layer "B.Cu") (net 27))
 (segment (start 120.5 112.8) (end 120.72 113.02) (width 0.2) (layer "B.Cu") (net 27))
 (segment (start 128.5 118) (end 128.42007 117.92007) (width 0.2) (layer "B.Cu") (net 27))
 (segment (start 128.42007 117.92007) (end 128.42007 115.92846) (width 0.2) (layer "B.Cu") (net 27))
 (segment (start 125.5 96) (end 126.8 97.3) (width 0.2) (layer "B.Cu") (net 27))
 (segment (start 120.72 113.02) (end 120.72 114.72) (width 0.2) (layer "B.Cu") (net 27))
 (segment (start 120.72 114.72) (end 123.5 117.5) (width 0.2) (layer "B.Cu") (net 27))
 (segment (start 125.5 94.96) (end 125.5 96) (width 0.2) (layer "B.Cu") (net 27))
 (segment (start 120.7 113) (end 120.5 112.8) (width 0.2) (layer "B.Cu") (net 27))
 (segment (start 126.8 97.3) (end 126.8 113) (width 0.2) (layer "B.Cu") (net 27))
 (segment (start 131.5 115) (end 130.9 115.6) (width 0.2) (layer "B.Cu") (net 27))
 (segment (start 121.3 163.36) (end 120.2 162.26) (width 0.2) (layer "F.Cu") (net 25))
 (segment (start 135.315635 163.86) (end 135.96 163.215635) (width 0.2) (layer "B.Cu") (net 25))
 (segment (start 121.74 163.86) (end 135.315635 163.86) (width 0.2) (layer "B.Cu") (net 25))
 (segment (start 120.64 162.76) (end 121.74 163.86) (width 0.2) (layer "B.Cu") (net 25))
 (segment (start 173.504365 124.76) (end 177.76 124.76) (width 0.2) (layer "B.Cu") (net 25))
 (segment (start 135.96 162.304365) (end 173.504365 124.76) (width 0.2) (layer "B.Cu") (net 25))
 (segment (start 135.96 163.215635) (end 135.96 162.304365) (width 0.2) (layer "B.Cu") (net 25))
 (segment (start 110.02 113.98) (end 110.04 114) (width 0.2) (layer "F.Cu") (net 21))
 (segment (start 101.84 105.8) (end 110.02 113.98) (width 0.2) (layer "F.Cu") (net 21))
 (segment (start 101.84 80.26) (end 101.84 105.8) (width 0.2) (layer "F.Cu") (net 21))
 (via (at 110.02 113.98) (size 0.6) (drill 0.3) (layers "F.Cu" "B.Cu") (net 21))
 (segment (start 132.32 162.76) (end 133.6 161.48) (width 0.2) (layer "B.Cu") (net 21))
 (segment (start 110.9 122.4) (end 110.9 114.834315) (width 0.2) (layer "B.Cu") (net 21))
 (segment (start 110.045685 113.98) (end 110.02 113.98) (width 0.2) (layer "B.Cu") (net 21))
 (segment (start 133.6 161.48) (end 133.6 145.1) (width 0.2) (layer "B.Cu") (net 21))
 (segment (start 110.9 114.834315) (end 110.045685 113.98) (width 0.2) (layer "B.Cu") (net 21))
 (segment (start 133.6 145.1) (end 110.9 122.4) (width 0.2) (layer "B.Cu") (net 21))
 (segment (start 102.02 114.165686) (end 115.620049 127.765735) (width 0.2) (layer "F.Cu") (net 20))
 (segment (start 107.8 114.7) (end 103.685686 114.7) (width 0.2) (layer "F.Cu") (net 20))
 (segment (start 109.46 80.26) (end 107.26 78.06) (width 0.2) (layer "F.Cu") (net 20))
 (segment (start 102.254314 113.6) (end 102.02 113.834314) (width 0.2) (layer "F.Cu") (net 20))
 (segment (start 101.23939 78.06) (end 100.19 79.10939) (width 0.2) (layer "F.Cu") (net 20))
 (segment (start 102.585686 113.6) (end 102.254314 113.6) (width 0.2) (layer "F.Cu") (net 20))
 (segment (start 100.19 79.10939) (end 100.19 108.5) (width 0.2) (layer "F.Cu") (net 20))
 (segment (start 103.685686 114.7) (end 102.585686 113.6) (width 0.2) (layer "F.Cu") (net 20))
 (segment (start 102.02 113.834314) (end 102.02 114.165686) (width 0.2) (layer "F.Cu") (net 20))
 (segment (start 107.26 78.06) (end 101.23939 78.06) (width 0.2) (layer "F.Cu") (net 20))
 (segment (start 108 114.5) (end 107.8 114.7) (width 0.2) (layer "F.Cu") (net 20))
 (segment (start 115.620049 127.765735) (end 117.265735 127.765735) (width 0.2) (layer "F.Cu") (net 20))
 (via (at 117.265735 127.765735) (size 0.6) (drill 0.3) (layers "F.Cu" "B.Cu") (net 20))
 (via (at 108 114.5) (size 0.6) (drill 0.3) (layers "F.Cu" "B.Cu") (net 20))
 (via (at 100.19 108.5) (size 0.6) (drill 0.3) (layers "F.Cu" "B.Cu") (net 20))
 (segment (start 107.5 114) (end 108 114.5) (width 0.2) (layer "B.Cu") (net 20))
 (segment (start 117.265735 127.765735) (end 134.86 145.36) (width 0.2) (layer "B.Cu") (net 20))
 (segment (start 100.19 108.5) (end 102 108.5) (width 0.2) (layer "B.Cu") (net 20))
 (segment (start 102 108.5) (end 107.5 114) (width 0.2) (layer "B.Cu") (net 20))
 (segment (start 134.86 145.36) (end 134.86 162.76) (width 0.2) (layer "B.Cu") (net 20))
 (segment (start 126.844365 116) (end 125.8 114.955635) (width 0.2) (layer "F.Cu") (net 24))
 (segment (start 158.68 95.56) (end 116.62 95.56) (width 0.2) (layer "F.Cu") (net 24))
 (segment (start 129.324365 113.4) (end 128.68 114.044365) (width 0.2) (layer "F.Cu") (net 24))
 (segment (start 131.845686 113.4) (end 129.324365 113.4) (width 0.2) (layer "F.Cu") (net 24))
 (segment (start 132.28 153.66) (end 132.28 113.834314) (width 0.2) (layer "F.Cu") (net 24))
 (segment (start 125.155635 113.4) (end 119.1 113.4) (width 0.2) (layer "F.Cu") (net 24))
 (segment (start 128.68 114.044365) (end 128.68 114.82) (width 0.2) (layer "F.Cu") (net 24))
 (segment (start 116.62 111.44) (end 118.84 113.66) (width 0.2) (layer "F.Cu") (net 24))
 (segment (start 119.1 113.4) (end 118.84 113.66) (width 0.2) (layer "F.Cu") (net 24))
 (segment (start 125.8 114.955635) (end 125.8 114.044365) (width 0.2) (layer "F.Cu") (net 24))
 (segment (start 116.62 95.56) (end 116.62 111.44) (width 0.2) (layer "F.Cu") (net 24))
 (segment (start 132.28 113.834314) (end 131.845686 113.4) (width 0.2) (layer "F.Cu") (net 24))
 (segment (start 184.36 97.76) (end 172.62 109.5) (width 0.2) (layer "F.Cu") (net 24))
 (segment (start 125.8 114.044365) (end 125.155635 113.4) (width 0.2) (layer "F.Cu") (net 24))
 (segment (start 128.68 114.82) (end 127.5 116) (width 0.2) (layer "F.Cu") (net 24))
 (segment (start 123.18 162.76) (end 132.28 153.66) (width 0.2) (layer "F.Cu") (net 24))
 (segment (start 127.5 116) (end 126.844365 116) (width 0.2) (layer "F.Cu") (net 24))
 (segment (start 184.36 91.04) (end 184.36 97.76) (width 0.2) (layer "F.Cu") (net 24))
 (segment (start 172.62 109.5) (end 158.68 95.56) (width 0.2) (layer "F.Cu") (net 24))
 (segment (start 185.36 124.76) (end 185.75 124.37) (width 0.2) (layer "F.Cu") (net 33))
 (segment (start 185.75 124.37) (end 185.75 94.4) (width 0.2) (layer "F.Cu") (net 33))
 (segment (start 184.86 125.26) (end 185.36 124.76) (width 0.2) (layer "F.Cu") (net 33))
 (segment (start 184.86 140.26) (end 184.86 125.26) (width 0.2) (layer "F.Cu") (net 33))
 (segment (start 117.82 96.76) (end 133.96 112.9) (width 0.2) (layer "F.Cu") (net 32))
 (segment (start 152.42 112.9) (end 179.78 140.26) (width 0.2) (layer "F.Cu") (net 32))
 (segment (start 133.96 112.9) (end 152.42 112.9) (width 0.2) (layer "F.Cu") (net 32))
 (segment (start 177.64 92.94) (end 178.5 93.8) (width 0.2) (layer "F.Cu") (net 45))
 (segment (start 177.64 91.04) (end 177.64 92.94) (width 0.2) (layer "F.Cu") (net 45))
 (via (at 178.5 93.8) (size 0.6) (drill 0.3) (layers "F.Cu" "B.Cu") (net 45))
 (segment (start 177.64 94.66) (end 177.64 97.76) (width 0.2) (layer "B.Cu") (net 45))
 (segment (start 178.5 93.8) (end 177.64 94.66) (width 0.2) (layer "B.Cu") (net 45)))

